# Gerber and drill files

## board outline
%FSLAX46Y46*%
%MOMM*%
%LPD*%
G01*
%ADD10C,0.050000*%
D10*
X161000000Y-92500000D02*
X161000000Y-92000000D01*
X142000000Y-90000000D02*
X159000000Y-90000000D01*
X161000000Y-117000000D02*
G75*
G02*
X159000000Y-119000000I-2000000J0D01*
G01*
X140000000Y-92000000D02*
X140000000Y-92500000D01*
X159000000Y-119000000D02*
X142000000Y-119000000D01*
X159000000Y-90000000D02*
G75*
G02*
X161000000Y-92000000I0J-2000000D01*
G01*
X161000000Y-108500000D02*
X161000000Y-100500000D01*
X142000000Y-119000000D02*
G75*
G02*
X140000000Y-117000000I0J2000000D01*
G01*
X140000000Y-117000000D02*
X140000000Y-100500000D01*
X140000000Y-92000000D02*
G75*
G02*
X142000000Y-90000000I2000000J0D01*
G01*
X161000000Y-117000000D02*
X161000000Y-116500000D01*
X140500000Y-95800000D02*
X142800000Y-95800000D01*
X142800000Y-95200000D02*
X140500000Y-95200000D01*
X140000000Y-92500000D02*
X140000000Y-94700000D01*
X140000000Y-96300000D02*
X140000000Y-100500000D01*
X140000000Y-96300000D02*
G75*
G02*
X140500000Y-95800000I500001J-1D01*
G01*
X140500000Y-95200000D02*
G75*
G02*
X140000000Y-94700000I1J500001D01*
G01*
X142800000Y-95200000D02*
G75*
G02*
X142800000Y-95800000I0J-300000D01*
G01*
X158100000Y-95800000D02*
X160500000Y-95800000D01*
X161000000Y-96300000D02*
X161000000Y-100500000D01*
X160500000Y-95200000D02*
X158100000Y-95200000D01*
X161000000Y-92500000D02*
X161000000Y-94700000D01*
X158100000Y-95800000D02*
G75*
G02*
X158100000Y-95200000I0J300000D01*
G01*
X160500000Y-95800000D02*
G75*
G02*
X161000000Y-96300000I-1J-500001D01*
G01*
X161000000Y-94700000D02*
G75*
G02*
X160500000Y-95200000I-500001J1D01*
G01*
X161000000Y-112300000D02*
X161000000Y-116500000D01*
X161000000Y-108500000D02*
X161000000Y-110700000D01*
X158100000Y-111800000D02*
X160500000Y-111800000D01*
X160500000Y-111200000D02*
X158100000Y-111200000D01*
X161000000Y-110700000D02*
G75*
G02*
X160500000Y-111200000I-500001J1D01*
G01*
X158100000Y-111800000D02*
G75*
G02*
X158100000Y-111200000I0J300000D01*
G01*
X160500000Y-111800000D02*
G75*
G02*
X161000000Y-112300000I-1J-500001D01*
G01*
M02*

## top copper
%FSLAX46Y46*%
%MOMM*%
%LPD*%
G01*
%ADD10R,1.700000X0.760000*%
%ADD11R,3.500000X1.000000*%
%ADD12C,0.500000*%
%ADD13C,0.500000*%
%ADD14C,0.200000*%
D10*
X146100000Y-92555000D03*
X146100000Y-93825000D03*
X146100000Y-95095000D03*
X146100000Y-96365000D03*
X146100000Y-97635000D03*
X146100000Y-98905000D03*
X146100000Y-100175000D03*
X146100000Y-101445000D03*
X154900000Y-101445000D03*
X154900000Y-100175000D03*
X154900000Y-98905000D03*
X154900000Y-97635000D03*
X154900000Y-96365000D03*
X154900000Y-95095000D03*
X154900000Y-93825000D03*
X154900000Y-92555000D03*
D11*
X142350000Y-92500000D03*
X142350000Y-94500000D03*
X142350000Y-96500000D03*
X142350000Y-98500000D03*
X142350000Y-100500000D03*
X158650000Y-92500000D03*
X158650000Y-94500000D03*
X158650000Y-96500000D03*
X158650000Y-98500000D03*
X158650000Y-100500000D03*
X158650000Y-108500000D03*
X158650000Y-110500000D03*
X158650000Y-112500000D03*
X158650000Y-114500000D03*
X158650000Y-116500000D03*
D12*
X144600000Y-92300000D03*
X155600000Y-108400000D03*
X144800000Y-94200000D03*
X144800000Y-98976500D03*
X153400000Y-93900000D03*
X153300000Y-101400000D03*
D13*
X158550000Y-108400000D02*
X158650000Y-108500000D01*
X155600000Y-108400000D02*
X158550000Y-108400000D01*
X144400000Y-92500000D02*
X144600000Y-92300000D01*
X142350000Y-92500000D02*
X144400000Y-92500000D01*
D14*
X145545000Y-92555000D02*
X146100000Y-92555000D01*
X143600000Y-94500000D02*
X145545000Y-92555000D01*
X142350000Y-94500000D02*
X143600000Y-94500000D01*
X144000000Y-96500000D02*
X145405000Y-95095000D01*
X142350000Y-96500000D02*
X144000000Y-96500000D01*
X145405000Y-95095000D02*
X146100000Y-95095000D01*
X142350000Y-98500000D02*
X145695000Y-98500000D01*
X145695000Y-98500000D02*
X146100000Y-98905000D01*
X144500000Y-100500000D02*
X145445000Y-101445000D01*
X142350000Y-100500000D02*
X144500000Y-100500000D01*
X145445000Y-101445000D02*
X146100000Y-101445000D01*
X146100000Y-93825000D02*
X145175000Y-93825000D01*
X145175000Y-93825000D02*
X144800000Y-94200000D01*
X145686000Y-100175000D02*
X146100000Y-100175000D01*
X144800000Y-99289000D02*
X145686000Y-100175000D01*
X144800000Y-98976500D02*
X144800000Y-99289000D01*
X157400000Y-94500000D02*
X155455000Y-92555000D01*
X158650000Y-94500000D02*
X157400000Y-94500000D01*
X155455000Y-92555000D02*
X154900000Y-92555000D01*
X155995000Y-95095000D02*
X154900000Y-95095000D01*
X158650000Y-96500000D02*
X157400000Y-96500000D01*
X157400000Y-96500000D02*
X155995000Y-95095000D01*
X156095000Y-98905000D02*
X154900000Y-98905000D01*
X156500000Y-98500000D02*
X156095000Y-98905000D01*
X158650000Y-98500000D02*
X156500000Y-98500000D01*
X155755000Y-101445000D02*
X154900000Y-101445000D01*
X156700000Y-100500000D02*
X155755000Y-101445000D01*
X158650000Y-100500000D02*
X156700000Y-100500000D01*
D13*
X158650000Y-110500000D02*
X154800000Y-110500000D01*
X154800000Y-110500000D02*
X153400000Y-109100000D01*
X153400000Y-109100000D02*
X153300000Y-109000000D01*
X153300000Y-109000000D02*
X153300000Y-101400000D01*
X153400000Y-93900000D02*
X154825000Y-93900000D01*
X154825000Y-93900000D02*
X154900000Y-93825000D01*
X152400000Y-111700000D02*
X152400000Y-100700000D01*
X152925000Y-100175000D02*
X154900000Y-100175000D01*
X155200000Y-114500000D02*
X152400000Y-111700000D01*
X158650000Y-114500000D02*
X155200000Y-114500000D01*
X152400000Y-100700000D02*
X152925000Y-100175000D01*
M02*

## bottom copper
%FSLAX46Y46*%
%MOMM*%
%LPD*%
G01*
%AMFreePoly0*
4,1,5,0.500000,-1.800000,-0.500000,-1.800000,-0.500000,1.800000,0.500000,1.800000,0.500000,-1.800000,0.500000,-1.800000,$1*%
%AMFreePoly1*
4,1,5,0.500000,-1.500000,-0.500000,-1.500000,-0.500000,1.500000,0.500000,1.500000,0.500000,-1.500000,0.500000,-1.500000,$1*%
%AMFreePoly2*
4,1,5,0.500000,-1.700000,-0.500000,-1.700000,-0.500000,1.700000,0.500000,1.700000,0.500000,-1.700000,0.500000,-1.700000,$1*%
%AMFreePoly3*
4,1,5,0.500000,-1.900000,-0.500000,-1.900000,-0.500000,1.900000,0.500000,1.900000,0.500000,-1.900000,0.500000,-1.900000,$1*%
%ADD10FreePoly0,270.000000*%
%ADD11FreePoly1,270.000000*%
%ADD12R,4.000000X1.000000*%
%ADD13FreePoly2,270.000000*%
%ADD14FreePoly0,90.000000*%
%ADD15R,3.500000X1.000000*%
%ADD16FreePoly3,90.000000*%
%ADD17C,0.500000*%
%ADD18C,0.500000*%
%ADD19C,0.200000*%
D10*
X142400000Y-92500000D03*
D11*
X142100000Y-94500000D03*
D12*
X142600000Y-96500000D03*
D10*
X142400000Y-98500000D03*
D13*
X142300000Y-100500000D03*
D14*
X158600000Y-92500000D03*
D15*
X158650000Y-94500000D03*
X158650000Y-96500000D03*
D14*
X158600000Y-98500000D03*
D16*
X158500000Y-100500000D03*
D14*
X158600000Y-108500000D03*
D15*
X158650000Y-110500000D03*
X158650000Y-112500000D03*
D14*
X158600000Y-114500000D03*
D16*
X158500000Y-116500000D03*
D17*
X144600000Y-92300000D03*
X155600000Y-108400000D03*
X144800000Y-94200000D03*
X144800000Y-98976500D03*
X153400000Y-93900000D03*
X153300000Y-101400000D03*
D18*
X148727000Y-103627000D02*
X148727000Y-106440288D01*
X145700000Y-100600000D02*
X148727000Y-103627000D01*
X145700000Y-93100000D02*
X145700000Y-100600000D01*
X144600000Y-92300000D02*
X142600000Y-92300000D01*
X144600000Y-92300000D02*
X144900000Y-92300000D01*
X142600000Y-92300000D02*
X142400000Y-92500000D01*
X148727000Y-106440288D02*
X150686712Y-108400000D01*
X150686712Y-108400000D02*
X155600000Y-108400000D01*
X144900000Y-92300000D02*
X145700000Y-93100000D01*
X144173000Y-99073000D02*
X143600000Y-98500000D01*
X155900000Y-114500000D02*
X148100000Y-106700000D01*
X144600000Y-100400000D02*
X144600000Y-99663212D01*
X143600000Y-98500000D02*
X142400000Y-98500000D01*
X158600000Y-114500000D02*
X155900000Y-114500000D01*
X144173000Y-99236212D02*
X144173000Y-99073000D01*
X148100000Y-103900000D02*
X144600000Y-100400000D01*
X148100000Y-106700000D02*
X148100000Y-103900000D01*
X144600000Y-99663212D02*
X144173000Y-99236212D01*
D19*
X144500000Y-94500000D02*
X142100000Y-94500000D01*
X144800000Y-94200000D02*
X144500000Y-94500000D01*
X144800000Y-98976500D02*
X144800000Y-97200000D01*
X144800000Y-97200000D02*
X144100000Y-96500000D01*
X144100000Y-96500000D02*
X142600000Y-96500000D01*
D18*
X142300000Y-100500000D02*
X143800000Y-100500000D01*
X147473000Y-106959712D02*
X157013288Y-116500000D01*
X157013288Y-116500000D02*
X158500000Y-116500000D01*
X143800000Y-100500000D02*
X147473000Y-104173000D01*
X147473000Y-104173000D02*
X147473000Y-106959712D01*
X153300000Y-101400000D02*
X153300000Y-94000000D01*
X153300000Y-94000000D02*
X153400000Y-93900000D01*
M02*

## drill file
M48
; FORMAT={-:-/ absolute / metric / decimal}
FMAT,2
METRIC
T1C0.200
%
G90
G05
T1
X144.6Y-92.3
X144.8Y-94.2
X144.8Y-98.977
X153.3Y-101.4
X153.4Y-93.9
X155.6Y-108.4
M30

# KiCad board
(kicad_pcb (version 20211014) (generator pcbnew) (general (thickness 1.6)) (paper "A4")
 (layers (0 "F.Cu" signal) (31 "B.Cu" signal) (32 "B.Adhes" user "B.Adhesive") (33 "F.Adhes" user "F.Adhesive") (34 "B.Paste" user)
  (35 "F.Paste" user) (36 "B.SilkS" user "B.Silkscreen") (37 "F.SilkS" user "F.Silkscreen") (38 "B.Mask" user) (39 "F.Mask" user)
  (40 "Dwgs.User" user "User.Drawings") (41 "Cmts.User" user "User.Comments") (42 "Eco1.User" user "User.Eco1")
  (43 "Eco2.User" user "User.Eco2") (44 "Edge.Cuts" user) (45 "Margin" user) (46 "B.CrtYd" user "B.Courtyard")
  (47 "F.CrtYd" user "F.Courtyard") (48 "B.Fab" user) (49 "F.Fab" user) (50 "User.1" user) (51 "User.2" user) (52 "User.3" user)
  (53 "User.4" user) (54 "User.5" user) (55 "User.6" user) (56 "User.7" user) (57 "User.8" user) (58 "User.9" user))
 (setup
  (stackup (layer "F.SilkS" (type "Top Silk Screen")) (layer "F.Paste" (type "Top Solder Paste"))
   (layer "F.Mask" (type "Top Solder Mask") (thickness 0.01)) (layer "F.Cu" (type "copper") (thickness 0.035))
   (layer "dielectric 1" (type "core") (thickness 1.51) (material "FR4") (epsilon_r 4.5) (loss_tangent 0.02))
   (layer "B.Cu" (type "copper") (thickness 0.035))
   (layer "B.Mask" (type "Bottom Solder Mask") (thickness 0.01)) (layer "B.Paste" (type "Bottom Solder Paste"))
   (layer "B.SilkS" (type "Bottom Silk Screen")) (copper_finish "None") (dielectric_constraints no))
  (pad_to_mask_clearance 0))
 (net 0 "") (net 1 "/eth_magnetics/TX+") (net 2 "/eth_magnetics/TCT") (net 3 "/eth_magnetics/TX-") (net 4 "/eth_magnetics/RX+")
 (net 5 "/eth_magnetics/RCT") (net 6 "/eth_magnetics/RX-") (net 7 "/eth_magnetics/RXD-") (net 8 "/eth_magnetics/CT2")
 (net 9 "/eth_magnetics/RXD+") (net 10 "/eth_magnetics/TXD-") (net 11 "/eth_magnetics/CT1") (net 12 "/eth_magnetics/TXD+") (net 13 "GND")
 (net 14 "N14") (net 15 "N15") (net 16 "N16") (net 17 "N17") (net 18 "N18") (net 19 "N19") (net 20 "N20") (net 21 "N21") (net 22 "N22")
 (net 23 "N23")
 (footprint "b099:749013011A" (layer "F.Cu") (at 150.5 97)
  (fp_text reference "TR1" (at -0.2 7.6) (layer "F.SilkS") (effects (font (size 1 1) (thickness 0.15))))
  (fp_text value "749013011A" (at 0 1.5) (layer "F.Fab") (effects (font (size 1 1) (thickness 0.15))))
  (pad "1" smd rect (at -4.4 -4.445) (size 1.7 0.76) (layers "F.Cu" "F.Paste" "F.Mask") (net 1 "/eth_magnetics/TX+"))
  (pad "2" smd rect (at -4.4 -3.175) (size 1.7 0.76) (layers "F.Cu" "F.Paste" "F.Mask") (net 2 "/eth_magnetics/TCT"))
  (pad "3" smd rect (at -4.4 -1.905) (size 1.7 0.76) (layers "F.Cu" "F.Paste" "F.Mask") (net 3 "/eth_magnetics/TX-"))
  (pad "4" smd rect (at -4.4 -0.635) (size 1.7 0.76) (layers "F.Cu" "F.Paste" "F.Mask"))
  (pad "5" smd rect (at -4.4 0.635) (size 1.7 0.76) (layers "F.Cu" "F.Paste" "F.Mask"))
  (pad "6" smd rect (at -4.4 1.905) (size 1.7 0.76) (layers "F.Cu" "F.Paste" "F.Mask") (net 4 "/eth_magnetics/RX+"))
  (pad "7" smd rect (at -4.4 3.175) (size 1.7 0.76) (layers "F.Cu" "F.Paste" "F.Mask") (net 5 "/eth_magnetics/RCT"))
  (pad "8" smd rect (at -4.4 4.445) (size 1.7 0.76) (layers "F.Cu" "F.Paste" "F.Mask") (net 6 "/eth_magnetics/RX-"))
  (pad "9" smd rect (at 4.4 4.445) (size 1.7 0.76) (layers "F.Cu" "F.Paste" "F.Mask") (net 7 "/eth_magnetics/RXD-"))
  (pad "10" smd rect (at 4.4 3.175) (size 1.7 0.76) (layers "F.Cu" "F.Paste" "F.Mask") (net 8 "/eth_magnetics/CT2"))
  (pad "11" smd rect (at 4.4 1.905) (size 1.7 0.76) (layers "F.Cu" "F.Paste" "F.Mask") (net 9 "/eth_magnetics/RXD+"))
  (pad "12" smd rect (at 4.4 0.635) (size 1.7 0.76) (layers "F.Cu" "F.Paste" "F.Mask"))
  (pad "13" smd rect (at 4.4 -0.635) (size 1.7 0.76) (layers "F.Cu" "F.Paste" "F.Mask"))
  (pad "14" smd rect (at 4.4 -1.905) (size 1.7 0.76) (layers "F.Cu" "F.Paste" "F.Mask") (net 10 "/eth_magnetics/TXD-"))
  (pad "15" smd rect (at 4.4 -3.175) (size 1.7 0.76) (layers "F.Cu" "F.Paste" "F.Mask") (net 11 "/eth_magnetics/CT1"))
  (pad "16" smd rect (at 4.4 -4.445) (size 1.7 0.76) (layers "F.Cu" "F.Paste" "F.Mask") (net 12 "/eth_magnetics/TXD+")))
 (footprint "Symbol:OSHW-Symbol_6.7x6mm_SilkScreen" (layer "F.Cu") (at 143.5 115.5)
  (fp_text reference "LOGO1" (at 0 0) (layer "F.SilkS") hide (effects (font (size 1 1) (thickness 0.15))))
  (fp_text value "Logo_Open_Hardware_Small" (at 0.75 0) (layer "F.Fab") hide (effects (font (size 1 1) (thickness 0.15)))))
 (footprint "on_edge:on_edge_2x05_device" (layer "F.Cu") (at 140 96.5 -90)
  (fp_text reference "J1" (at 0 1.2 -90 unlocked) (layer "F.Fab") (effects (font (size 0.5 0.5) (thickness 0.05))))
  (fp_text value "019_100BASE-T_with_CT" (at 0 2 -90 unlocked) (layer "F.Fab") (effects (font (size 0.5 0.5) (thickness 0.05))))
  (fp_line (start -0.7 -0.5) (end -0.7 -2.8) (layer "Edge.Cuts") (width 0.05))
  (fp_line (start -1.3 -2.8) (end -1.3 -0.5) (layer "Edge.Cuts") (width 0.05))
  (fp_line (start -4 0) (end -1.8 0) (layer "Edge.Cuts") (width 0.05))
  (fp_line (start -0.2 0) (end 4 0) (layer "Edge.Cuts") (width 0.05))
  (fp_arc (start -0.2 0) (mid -0.553553 -0.146447) (end -0.7 -0.5) (layer "Edge.Cuts") (width 0.05))
  (fp_arc (start -1.3 -0.5) (mid -1.446447 -0.146447) (end -1.8 0) (layer "Edge.Cuts") (width 0.05))
  (fp_arc (start -1.3 -2.8) (mid -1 -3.1) (end -0.7 -2.8) (layer "Edge.Cuts") (width 0.05))
  (pad "1" smd rect (at -4 -2.35 90) (size 1 3.5) (layers "F.Cu" "F.Mask") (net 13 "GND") (zone_connect 0))
  (pad "2" smd rect (at -2 -2.35 270) (size 1 3.5) (layers "F.Cu" "F.Mask") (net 1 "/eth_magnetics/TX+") (zone_connect 0))
  (pad "3" smd rect (at 0 -2.35 270) (size 1 3.5) (layers "F.Cu" "F.Mask") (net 3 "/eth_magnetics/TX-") (zone_connect 0))
  (pad "4" smd rect (at 2 -2.35 90) (size 1 3.5) (layers "F.Cu" "F.Mask") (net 4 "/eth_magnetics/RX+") (zone_connect 0))
  (pad "5" smd rect (at 4 -2.35 90) (size 1 3.5) (layers "F.Cu" "F.Mask") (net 6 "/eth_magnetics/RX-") (zone_connect 0))
  (pad "6" smd custom (at -4 -2.4 270) (size 1 3.6) (layers "B.Cu" "B.Mask") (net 13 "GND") (zone_connect 0)
   (options (clearance outline) (anchor rect)) (primitives))
  (pad "7" smd custom (at -2 -2.1 270) (size 1 3) (layers "B.Cu" "B.Mask") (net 2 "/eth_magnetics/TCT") (zone_connect 0)
   (options (clearance outline) (anchor rect)) (primitives))
  (pad "8" smd rect (at 0 -2.6 270) (size 1 4) (layers "B.Cu" "B.Mask") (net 5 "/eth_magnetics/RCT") (zone_connect 0))
  (pad "9" smd custom (at 2 -2.4 270) (size 1 3.6) (layers "B.Cu" "B.Mask") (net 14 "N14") (zone_connect 0)
   (options (clearance outline) (anchor rect)) (primitives))
  (pad "10" smd custom (at 4 -2.3 270) (size 1 3.4) (layers "B.Cu" "B.Mask") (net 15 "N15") (zone_connect 0)
   (options (clearance outline) (anchor rect)) (primitives))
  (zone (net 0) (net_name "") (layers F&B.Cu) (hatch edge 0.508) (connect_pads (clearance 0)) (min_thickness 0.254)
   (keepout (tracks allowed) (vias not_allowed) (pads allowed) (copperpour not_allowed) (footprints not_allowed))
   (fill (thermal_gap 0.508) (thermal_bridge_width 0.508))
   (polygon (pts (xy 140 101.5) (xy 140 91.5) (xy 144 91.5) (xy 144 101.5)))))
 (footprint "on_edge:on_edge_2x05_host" (layer "F.Cu") (at 161 96.5 -90)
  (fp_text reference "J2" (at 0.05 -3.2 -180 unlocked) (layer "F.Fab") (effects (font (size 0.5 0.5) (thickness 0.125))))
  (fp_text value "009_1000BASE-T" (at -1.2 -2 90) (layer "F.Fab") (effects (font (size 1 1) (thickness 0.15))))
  (fp_line (start -0.7 2.9) (end -0.7 0.5) (layer "Edge.Cuts") (width 0.05))
  (fp_line (start -0.2 0) (end 4 0) (layer "Edge.Cuts") (width 0.05))
  (fp_line (start -1.3 0.5) (end -1.3 2.9) (layer "Edge.Cuts") (width 0.05))
  (fp_line (start -4 0) (end -1.8 0) (layer "Edge.Cuts") (width 0.05))
  (fp_arc (start -0.7 2.9) (mid -1 3.2) (end -1.3 2.9) (layer "Edge.Cuts") (width 0.05))
  (fp_arc (start -0.7 0.5) (mid -0.553553 0.146447) (end -0.2 0) (layer "Edge.Cuts") (width 0.05))
  (fp_arc (start -1.8 0) (mid -1.446447 0.146447) (end -1.3 0.5) (layer "Edge.Cuts") (width 0.05))
  (pad "1" smd rect (at -4 2.35 270) (size 1 3.5) (layers "F.Cu" "F.Mask") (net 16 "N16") (zone_connect 0))
  (pad "2" smd rect (at -2 2.35 270) (size 1 3.5) (layers "F.Cu" "F.Mask") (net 12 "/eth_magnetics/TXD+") (zone_connect 0))
  (pad "3" smd rect (at 0 2.35 270) (size 1 3.5) (layers "F.Cu" "F.Mask") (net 10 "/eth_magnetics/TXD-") (zone_connect 0))
  (pad "4" smd rect (at 2 2.35 270) (size 1 3.5) (layers "F.Cu" "F.Mask") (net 9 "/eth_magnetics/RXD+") (zone_connect 0))
  (pad "5" smd rect (at 4 2.35 270) (size 1 3.5) (layers "F.Cu" "F.Mask") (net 7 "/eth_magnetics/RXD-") (zone_connect 0))
  (pad "6" smd custom (at -4 2.4 90) (size 1 3.6) (layers "B.Cu" "B.Mask") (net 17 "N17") (zone_connect 0)
   (options (clearance outline) (anchor rect)) (primitives))
  (pad "7" smd rect (at -2 2.35 90) (size 1 3.5) (layers "B.Cu" "B.Mask") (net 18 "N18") (zone_connect 0))
  (pad "8" smd rect (at 0 2.35 90) (size 1 3.5) (layers "B.Cu" "B.Mask") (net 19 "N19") (zone_connect 0))
  (pad "9" smd custom (at 2 2.4 90) (size 1 3.6) (layers "B.Cu" "B.Mask") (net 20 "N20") (zone_connect 0)
   (options (clearance outline) (anchor rect)) (primitives))
  (pad "10" smd custom (at 4 2.5 90) (size 1 3.8) (layers "B.Cu" "B.Mask") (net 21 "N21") (zone_connect 0)
   (options (clearance outline) (anchor rect)) (primitives))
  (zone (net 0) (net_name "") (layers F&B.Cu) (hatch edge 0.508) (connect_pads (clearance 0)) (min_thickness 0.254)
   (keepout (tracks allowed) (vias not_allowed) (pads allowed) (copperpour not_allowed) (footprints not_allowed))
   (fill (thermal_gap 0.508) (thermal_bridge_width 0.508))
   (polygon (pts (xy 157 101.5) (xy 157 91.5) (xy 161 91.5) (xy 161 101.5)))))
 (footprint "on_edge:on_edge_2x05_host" (layer "F.Cu") (at 161 112.5 -90)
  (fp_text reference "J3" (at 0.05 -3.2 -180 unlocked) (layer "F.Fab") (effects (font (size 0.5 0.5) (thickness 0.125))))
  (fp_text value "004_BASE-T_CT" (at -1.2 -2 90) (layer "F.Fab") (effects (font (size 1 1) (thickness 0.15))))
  (fp_line (start -0.2 0) (end 4 0) (layer "Edge.Cuts") (width 0.05))
  (fp_line (start -4 0) (end -1.8 0) (layer "Edge.Cuts") (width 0.05))
  (fp_line (start -0.7 2.9) (end -0.7 0.5) (layer "Edge.Cuts") (width 0.05))
  (fp_line (start -1.3 0.5) (end -1.3 2.9) (layer "Edge.Cuts") (width 0.05))
  (fp_arc (start -1.8 0) (mid -1.446447 0.146447) (end -1.3 0.5) (layer "Edge.Cuts") (width 0.05))
  (fp_arc (start -0.7 2.9) (mid -1 3.2) (end -1.3 2.9) (layer "Edge.Cuts") (width 0.05))
  (fp_arc (start -0.7 0.5) (mid -0.553553 0.146447) (end -0.2 0) (layer "Edge.Cuts") (width 0.05))
  (pad "1" smd rect (at -4 2.35 270) (size 1 3.5) (layers "F.Cu" "F.Mask") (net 13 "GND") (zone_connect 0))
  (pad "2" smd rect (at -2 2.35 270) (size 1 3.5) (layers "F.Cu" "F.Mask") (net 11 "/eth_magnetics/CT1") (zone_connect 0))
  (pad "3" smd rect (at 0 2.35 270) (size 1 3.5) (layers "F.Cu" "F.Mask") (zone_connect 0))
  (pad "4" smd rect (at 2 2.35 270) (size 1 3.5) (layers "F.Cu" "F.Mask") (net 8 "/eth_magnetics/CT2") (zone_connect 0))
  (pad "5" smd rect (at 4 2.35 270) (size 1 3.5) (layers "F.Cu" "F.Mask") (zone_connect 0))
  (pad "6" smd custom (at -4 2.4 90) (size 1 3.6) (layers "B.Cu" "B.Mask") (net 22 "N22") (zone_connect 0)
   (options (clearance outline) (anchor rect)) (primitives))
  (pad "7" smd rect (at -2 2.35 90) (size 1 3.5) (layers "B.Cu" "B.Mask") (zone_connect 0))
  (pad "8" smd rect (at 0 2.35 90) (size 1 3.5) (layers "B.Cu" "B.Mask") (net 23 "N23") (zone_connect 0))
  (pad "9" smd custom (at 2 2.4 90) (size 1 3.6) (layers "B.Cu" "B.Mask") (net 14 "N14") (zone_connect 0)
   (options (clearance outline) (anchor rect)) (primitives))
  (pad "10" smd custom (at 4 2.5 90) (size 1 3.8) (layers "B.Cu" "B.Mask") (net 15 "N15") (zone_connect 0)
   (options (clearance outline) (anchor rect)) (primitives))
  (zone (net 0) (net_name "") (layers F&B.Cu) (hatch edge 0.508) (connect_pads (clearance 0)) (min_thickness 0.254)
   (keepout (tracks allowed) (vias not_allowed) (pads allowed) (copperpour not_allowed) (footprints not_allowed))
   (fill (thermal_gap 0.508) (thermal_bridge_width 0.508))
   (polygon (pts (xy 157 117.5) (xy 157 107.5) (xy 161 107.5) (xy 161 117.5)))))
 (gr_line (start 161 92.5) (end 161 92) (layer "Edge.Cuts") (width 0.05))
 (gr_line (start 142 90) (end 159 90) (layer "Edge.Cuts") (width 0.05))
 (gr_arc (start 161 117) (mid 160.414214 118.414214) (end 159 119) (layer "Edge.Cuts") (width 0.05))
 (gr_line (start 140 92) (end 140 92.5) (layer "Edge.Cuts") (width 0.05))
 (gr_line (start 159 119) (end 142 119) (layer "Edge.Cuts") (width 0.05))
 (gr_arc (start 159 90) (mid 160.414214 90.585786) (end 161 92) (layer "Edge.Cuts") (width 0.05))
 (gr_line (start 161 108.5) (end 161 100.5) (layer "Edge.Cuts") (width 0.05))
 (gr_arc (start 142 119) (mid 140.585786 118.414214) (end 140 117) (layer "Edge.Cuts") (width 0.05))
 (gr_line (start 140 117) (end 140 100.5) (layer "Edge.Cuts") (width 0.05))
 (gr_arc (start 140 92) (mid 140.585786 90.585786) (end 142 90) (layer "Edge.Cuts") (width 0.05))
 (gr_line (start 161 117) (end 161 116.5) (layer "Edge.Cuts") (width 0.05))
 (segment (start 158.55 108.4) (end 158.65 108.5) (width 0.5) (layer "F.Cu") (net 13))
 (segment (start 155.6 108.4) (end 158.55 108.4) (width 0.5) (layer "F.Cu") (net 13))
 (segment (start 144.4 92.5) (end 144.6 92.3) (width 0.5) (layer "F.Cu") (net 13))
 (segment (start 142.35 92.5) (end 144.4 92.5) (width 0.5) (layer "F.Cu") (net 13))
 (via (at 144.6 92.3) (size 0.5) (drill 0.2) (layers "F.Cu" "B.Cu") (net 13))
 (via (at 155.6 108.4) (size 0.5) (drill 0.2) (layers "F.Cu" "B.Cu") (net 13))
 (segment (start 148.727 103.627) (end 148.727 106.440288) (width 0.5) (layer "B.Cu") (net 13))
 (segment (start 145.7 100.6) (end 148.727 103.627) (width 0.5) (layer "B.Cu") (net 13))
 (segment (start 145.7 93.1) (end 145.7 100.6) (width 0.5) (layer "B.Cu") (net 13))
 (segment (start 144.6 92.3) (end 142.6 92.3) (width 0.5) (layer "B.Cu") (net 13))
 (segment (start 144.6 92.3) (end 144.9 92.3) (width 0.5) (layer "B.Cu") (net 13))
 (segment (start 142.6 92.3) (end 142.4 92.5) (width 0.5) (layer "B.Cu") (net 13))
 (segment (start 148.727 106.440288) (end 150.686712 108.4) (width 0.5) (layer "B.Cu") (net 13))
 (segment (start 150.686712 108.4) (end 155.6 108.4) (width 0.5) (layer "B.Cu") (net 13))
 (segment (start 144.9 92.3) (end 145.7 93.1) (width 0.5) (layer "B.Cu") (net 13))
 (segment (start 145.545 92.555) (end 146.1 92.555) (width 0.2) (layer "F.Cu") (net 1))
 (segment (start 143.6 94.5) (end 145.545 92.555) (width 0.2) (layer "F.Cu") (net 1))
 (segment (start 142.35 94.5) (end 143.6 94.5) (width 0.2) (layer "F.Cu") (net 1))
 (segment (start 144 96.5) (end 145.405 95.095) (width 0.2) (layer "F.Cu") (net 3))
 (segment (start 142.35 96.5) (end 144 96.5) (width 0.2) (layer "F.Cu") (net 3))
 (segment (start 145.405 95.095) (end 146.1 95.095) (width 0.2) (layer "F.Cu") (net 3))
 (segment (start 142.35 98.5) (end 145.695 98.5) (width 0.2) (layer "F.Cu") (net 4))
 (segment (start 145.695 98.5) (end 146.1 98.905) (width 0.2) (layer "F.Cu") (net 4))
 (segment (start 144.5 100.5) (end 145.445 101.445) (width 0.2) (layer "F.Cu") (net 6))
 (segment (start 142.35 100.5) (end 144.5 100.5) (width 0.2) (layer "F.Cu") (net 6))
 (segment (start 145.445 101.445) (end 146.1 101.445) (width 0.2) (layer "F.Cu") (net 6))
 (segment (start 144.173 99.073) (end 143.6 98.5) (width 0.5) (layer "B.Cu") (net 14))
 (segment (start 155.9 114.5) (end 148.1 106.7) (width 0.5) (layer "B.Cu") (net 14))
 (segment (start 144.6 100.4) (end 144.6 99.663212) (width 0.5) (layer "B.Cu") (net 14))
 (segment (start 143.6 98.5) (end 142.4 98.5) (width 0.5) (layer "B.Cu") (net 14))
 (segment (start 158.6 114.5) (end 155.9 114.5) (width 0.5) (layer "B.Cu") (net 14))
 (segment (start 144.173 99.236212) (end 144.173 99.073) (width 0.5) (layer "B.Cu") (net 14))
 (segment (start 148.1 103.9) (end 144.6 100.4) (width 0.5) (layer "B.Cu") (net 14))
 (segment (start 148.1 106.7) (end 148.1 103.9) (width 0.5) (layer "B.Cu") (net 14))
 (segment (start 144.6 99.663212) (end 144.173 99.236212) (width 0.5) (layer "B.Cu") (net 14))
 (segment (start 146.1 93.825) (end 145.175 93.825) (width 0.2) (layer "F.Cu") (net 2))
 (segment (start 145.175 93.825) (end 144.8 94.2) (width 0.2) (layer "F.Cu") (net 2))
 (via (at 144.8 94.2) (size 0.5) (drill 0.2) (layers "F.Cu" "B.Cu") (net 2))
 (segment (start 144.5 94.5) (end 142.1 94.5) (width 0.2) (layer "B.Cu") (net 2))
 (segment (start 144.8 94.2) (end 144.5 94.5) (width 0.2) (layer "B.Cu") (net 2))
 (segment (start 145.686 100.175) (end 146.1 100.175) (width 0.2) (layer "F.Cu") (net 5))
 (segment (start 144.8 99.289) (end 145.686 100.175) (width 0.2) (layer "F.Cu") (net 5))
 (segment (start 144.8 98.9765) (end 144.8 99.289) (width 0.2) (layer "F.Cu") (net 5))
 (via (at 144.8 98.9765) (size 0.5) (drill 0.2) (layers "F.Cu" "B.Cu") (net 5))
 (segment (start 144.8 98.9765) (end 144.8 97.2) (width 0.2) (layer "B.Cu") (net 5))
 (segment (start 144.8 97.2) (end 144.1 96.5) (width 0.2) (layer "B.Cu") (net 5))
 (segment (start 144.1 96.5) (end 142.6 96.5) (width 0.2) (layer "B.Cu") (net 5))
 (segment (start 157.4 94.5) (end 155.455 92.555) (width 0.2) (layer "F.Cu") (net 12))
 (segment (start 158.65 94.5) (end 157.4 94.5) (width 0.2) (layer "F.Cu") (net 12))
 (segment (start 155.455 92.555) (end 154.9 92.555) (width 0.2) (layer "F.Cu") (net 12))
 (segment (start 155.995 95.095) (end 154.9 95.095) (width 0.2) (layer "F.Cu") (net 10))
 (segment (start 158.65 96.5) (end 157.4 96.5) (width 0.2) (layer "F.Cu") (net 10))
 (segment (start 157.4 96.5) (end 155.995 95.095) (width 0.2) (layer "F.Cu") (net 10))
 (segment (start 156.095 98.905) (end 154.9 98.905) (width 0.2) (layer "F.Cu") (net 9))
 (segment (start 156.5 98.5) (end 156.095 98.905) (width 0.2) (layer "F.Cu") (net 9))
 (segment (start 158.65 98.5) (end 156.5 98.5) (width 0.2) (layer "F.Cu") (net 9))
 (segment (start 155.755 101.445) (end 154.9 101.445) (width 0.2) (layer "F.Cu") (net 7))
 (segment (start 156.7 100.5) (end 155.755 101.445) (width 0.2) (layer "F.Cu") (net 7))
 (segment (start 158.65 100.5) (end 156.7 100.5) (width 0.2) (layer "F.Cu") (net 7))
 (segment (start 142.3 100.5) (end 143.8 100.5) (width 0.5) (layer "B.Cu") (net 15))
 (segment (start 147.473 106.959712) (end 157.013288 116.5) (width 0.5) (layer "B.Cu") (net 15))
 (segment (start 157.013288 116.5) (end 158.5 116.5) (width 0.5) (layer "B.Cu") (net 15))
 (segment (start 143.8 100.5) (end 147.473 104.173) (width 0.5) (layer "B.Cu") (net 15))
 (segment (start 147.473 104.173) (end 147.473 106.959712) (width 0.5) (layer "B.Cu") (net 15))
 (segment (start 158.65 110.5) (end 154.8 110.5) (width 0.5) (layer "F.Cu") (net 11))
 (segment (start 154.8 110.5) (end 153.4 109.1) (width 0.5) (layer "F.Cu") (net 11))
 (segment (start 153.4 109.1) (end 153.3 109) (width 0.5) (layer "F.Cu") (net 11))
 (segment (start 153.3 109) (end 153.3 101.4) (width 0.5) (layer "F.Cu") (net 11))
 (segment (start 153.4 93.9) (end 154.825 93.9) (width 0.5) (layer "F.Cu") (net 11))
 (segment (start 154.825 93.9) (end 154.9 93.825) (width 0.5) (layer "F.Cu") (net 11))
 (via (at 153.4 93.9) (size 0.5) (drill 0.2) (layers "F.Cu" "B.Cu") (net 11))
 (via (at 153.3 101.4) (size 0.5) (drill 0.2) (layers "F.Cu" "B.Cu") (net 11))
 (segment (start 153.3 101.4) (end 153.3 94) (width 0.5) (layer "B.Cu") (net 11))
 (segment (start 153.3 94) (end 153.4 93.9) (width 0.5) (layer "B.Cu") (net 11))
 (segment (start 152.4 111.7) (end 152.4 100.7) (width 0.5) (layer "F.Cu") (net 8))
 (segment (start 152.925 100.175) (end 154.9 100.175) (width 0.5) (layer "F.Cu") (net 8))
 (segment (start 155.2 114.5) (end 152.4 111.7) (width 0.5) (layer "F.Cu") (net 8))
 (segment (start 158.65 114.5) (end 155.2 114.5) (width 0.5) (layer "F.Cu") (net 8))
 (segment (start 152.4 100.7) (end 152.925 100.175) (width 0.5) (layer "F.Cu") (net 8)))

